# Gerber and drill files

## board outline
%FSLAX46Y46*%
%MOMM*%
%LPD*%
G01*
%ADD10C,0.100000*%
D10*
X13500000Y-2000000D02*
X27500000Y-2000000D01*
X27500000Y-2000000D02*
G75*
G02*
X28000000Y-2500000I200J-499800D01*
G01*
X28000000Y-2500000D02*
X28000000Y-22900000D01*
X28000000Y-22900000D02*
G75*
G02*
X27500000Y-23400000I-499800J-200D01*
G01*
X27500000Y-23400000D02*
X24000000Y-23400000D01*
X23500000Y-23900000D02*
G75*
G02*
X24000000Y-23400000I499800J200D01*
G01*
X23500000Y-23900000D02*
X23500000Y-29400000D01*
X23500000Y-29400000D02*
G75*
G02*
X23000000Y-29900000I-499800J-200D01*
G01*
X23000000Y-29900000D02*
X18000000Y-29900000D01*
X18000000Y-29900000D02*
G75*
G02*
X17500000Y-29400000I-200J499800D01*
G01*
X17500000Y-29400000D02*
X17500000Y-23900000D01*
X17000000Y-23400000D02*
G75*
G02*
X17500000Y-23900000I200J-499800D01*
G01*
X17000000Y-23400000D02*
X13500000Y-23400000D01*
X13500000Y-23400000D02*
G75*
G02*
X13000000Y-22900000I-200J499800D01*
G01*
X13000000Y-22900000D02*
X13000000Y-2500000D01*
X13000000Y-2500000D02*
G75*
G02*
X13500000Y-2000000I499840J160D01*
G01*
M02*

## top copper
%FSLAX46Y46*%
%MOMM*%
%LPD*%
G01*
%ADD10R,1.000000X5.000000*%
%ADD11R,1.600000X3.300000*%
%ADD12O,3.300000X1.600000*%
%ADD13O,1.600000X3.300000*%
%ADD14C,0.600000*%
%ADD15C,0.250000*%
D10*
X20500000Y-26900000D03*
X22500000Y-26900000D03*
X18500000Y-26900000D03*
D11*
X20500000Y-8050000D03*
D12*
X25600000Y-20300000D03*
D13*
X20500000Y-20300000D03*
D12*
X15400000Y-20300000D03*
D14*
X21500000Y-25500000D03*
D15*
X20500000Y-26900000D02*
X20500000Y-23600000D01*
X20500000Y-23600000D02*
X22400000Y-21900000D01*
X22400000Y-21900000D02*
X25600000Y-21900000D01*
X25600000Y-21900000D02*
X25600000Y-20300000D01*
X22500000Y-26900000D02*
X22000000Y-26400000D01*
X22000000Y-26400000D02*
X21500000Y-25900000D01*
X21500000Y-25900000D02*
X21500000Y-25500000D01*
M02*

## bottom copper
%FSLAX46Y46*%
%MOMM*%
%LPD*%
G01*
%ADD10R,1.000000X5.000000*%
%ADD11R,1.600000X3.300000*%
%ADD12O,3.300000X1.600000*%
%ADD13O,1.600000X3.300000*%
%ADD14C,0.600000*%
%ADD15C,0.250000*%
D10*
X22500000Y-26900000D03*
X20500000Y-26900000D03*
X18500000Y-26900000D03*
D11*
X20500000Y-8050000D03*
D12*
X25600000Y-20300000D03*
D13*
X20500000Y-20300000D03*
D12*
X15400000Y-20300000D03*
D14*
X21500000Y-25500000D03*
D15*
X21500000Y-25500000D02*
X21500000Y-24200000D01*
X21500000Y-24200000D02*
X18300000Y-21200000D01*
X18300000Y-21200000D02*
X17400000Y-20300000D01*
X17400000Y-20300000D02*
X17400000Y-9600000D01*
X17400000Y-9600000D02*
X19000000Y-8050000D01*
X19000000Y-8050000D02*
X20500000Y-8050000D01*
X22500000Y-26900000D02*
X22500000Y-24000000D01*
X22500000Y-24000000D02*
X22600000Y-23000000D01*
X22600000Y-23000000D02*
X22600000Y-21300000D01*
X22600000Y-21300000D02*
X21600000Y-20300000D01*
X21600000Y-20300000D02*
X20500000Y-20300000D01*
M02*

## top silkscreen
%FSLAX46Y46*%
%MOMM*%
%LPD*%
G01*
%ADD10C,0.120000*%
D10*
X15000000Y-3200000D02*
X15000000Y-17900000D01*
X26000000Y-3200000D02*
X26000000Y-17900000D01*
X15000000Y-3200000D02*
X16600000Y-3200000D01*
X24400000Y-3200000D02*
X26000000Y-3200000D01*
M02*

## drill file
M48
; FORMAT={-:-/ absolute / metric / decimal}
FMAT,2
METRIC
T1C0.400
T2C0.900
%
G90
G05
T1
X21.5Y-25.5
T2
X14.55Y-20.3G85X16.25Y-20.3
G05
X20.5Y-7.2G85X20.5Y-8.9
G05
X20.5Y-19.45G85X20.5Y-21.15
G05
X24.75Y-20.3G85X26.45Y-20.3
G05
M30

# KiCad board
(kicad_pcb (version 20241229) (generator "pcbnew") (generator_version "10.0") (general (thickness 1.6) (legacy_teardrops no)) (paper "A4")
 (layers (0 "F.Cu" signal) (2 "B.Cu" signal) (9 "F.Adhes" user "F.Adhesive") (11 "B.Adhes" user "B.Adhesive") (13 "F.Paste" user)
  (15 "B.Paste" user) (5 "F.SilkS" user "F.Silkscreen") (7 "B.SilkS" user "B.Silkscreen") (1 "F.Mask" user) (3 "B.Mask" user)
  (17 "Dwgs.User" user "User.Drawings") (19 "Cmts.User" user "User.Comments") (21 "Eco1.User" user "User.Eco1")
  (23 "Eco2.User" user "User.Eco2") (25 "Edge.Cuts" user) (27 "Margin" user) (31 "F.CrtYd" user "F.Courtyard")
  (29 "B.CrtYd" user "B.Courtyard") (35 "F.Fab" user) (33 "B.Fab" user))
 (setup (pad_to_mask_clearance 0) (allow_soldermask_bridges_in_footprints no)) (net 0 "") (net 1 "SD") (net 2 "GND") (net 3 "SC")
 (gr_line (start 13.5 2.0) (end 27.5 2.0) (stroke (width 0.1) (type default)) (layer "Edge.Cuts"))
 (gr_arc (start 27.5 2.0) (mid 27.8536 2.1464) (end 28.0 2.5) (stroke (width 0.1) (type default)) (layer "Edge.Cuts"))
 (gr_line (start 28.0 2.5) (end 28.0 22.9) (stroke (width 0.1) (type default)) (layer "Edge.Cuts"))
 (gr_arc (start 28.0 22.9) (mid 27.8536 23.2536) (end 27.5 23.4) (stroke (width 0.1) (type default)) (layer "Edge.Cuts"))
 (gr_line (start 27.5 23.4) (end 24.0 23.4) (stroke (width 0.1) (type default)) (layer "Edge.Cuts"))
 (gr_arc (start 24.0 23.4) (mid 23.6464 23.5464) (end 23.5 23.9) (stroke (width 0.1) (type default)) (layer "Edge.Cuts"))
 (gr_line (start 23.5 23.9) (end 23.5 29.4) (stroke (width 0.1) (type default)) (layer "Edge.Cuts"))
 (gr_arc (start 23.5 29.4) (mid 23.3536 29.7536) (end 23.0 29.9) (stroke (width 0.1) (type default)) (layer "Edge.Cuts"))
 (gr_line (start 23.0 29.9) (end 18.0 29.9) (stroke (width 0.1) (type default)) (layer "Edge.Cuts"))
 (gr_arc (start 18.0 29.9) (mid 17.6464 29.7536) (end 17.5 29.4) (stroke (width 0.1) (type default)) (layer "Edge.Cuts"))
 (gr_line (start 17.5 29.4) (end 17.5 23.9) (stroke (width 0.1) (type default)) (layer "Edge.Cuts"))
 (gr_arc (start 17.5 23.9) (mid 17.3536 23.5464) (end 17.0 23.4) (stroke (width 0.1) (type default)) (layer "Edge.Cuts"))
 (gr_line (start 17.0 23.4) (end 13.5 23.4) (stroke (width 0.1) (type default)) (layer "Edge.Cuts"))
 (gr_arc (start 13.5 23.4) (mid 13.1464 23.2536) (end 13.0 22.9) (stroke (width 0.1) (type default)) (layer "Edge.Cuts"))
 (gr_line (start 13.0 22.9) (end 13.0 2.5) (stroke (width 0.1) (type default)) (layer "Edge.Cuts"))
 (gr_arc (start 13.0 2.5) (mid 13.1464 2.1464) (end 13.5 2.0) (stroke (width 0.1) (type default)) (layer "Edge.Cuts"))
 (gr_line (start 15.0 3.2) (end 15.0 17.9) (stroke (width 0.12) (type default)) (layer "F.SilkS"))
 (gr_line (start 26.0 3.2) (end 26.0 17.9) (stroke (width 0.12) (type default)) (layer "F.SilkS"))
 (gr_line (start 15.0 3.2) (end 16.6 3.2) (stroke (width 0.12) (type default)) (layer "F.SilkS"))
 (gr_line (start 24.4 3.2) (end 26.0 3.2) (stroke (width 0.12) (type default)) (layer "F.SilkS"))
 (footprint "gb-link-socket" (layer "F.Cu") (at 20.5 26.9)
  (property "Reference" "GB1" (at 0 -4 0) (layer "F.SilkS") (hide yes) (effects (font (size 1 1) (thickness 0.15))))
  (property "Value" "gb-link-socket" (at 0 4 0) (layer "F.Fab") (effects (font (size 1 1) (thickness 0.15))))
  (pad "4" smd rect (at 0 0) (size 1 5) (layers "F.Cu" "F.Mask") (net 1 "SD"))
  (pad "6" smd rect (at 2 0) (size 1 5) (layers "F.Cu" "F.Mask") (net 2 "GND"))
  (pad "2" smd rect (at -2 0) (size 1 5) (layers "F.Cu" "F.Mask"))
  (pad "5" smd rect (at 2 0) (size 1 5) (layers "B.Cu" "B.Mask") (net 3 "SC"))
  (pad "3" smd rect (at 0 0) (size 1 5) (layers "B.Cu" "B.Mask"))
  (pad "1" smd rect (at -2 0) (size 1 5) (layers "B.Cu" "B.Mask")))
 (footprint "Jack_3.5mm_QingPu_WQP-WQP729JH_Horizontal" (layer "F.Cu") (at 20.5 2.0 270)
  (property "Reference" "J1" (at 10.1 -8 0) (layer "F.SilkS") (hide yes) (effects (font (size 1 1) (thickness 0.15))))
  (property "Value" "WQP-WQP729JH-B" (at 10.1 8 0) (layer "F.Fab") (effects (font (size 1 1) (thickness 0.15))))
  (pad "1" thru_hole rect (at 6.05 0) (size 1.6 3.3) (drill oval 0.9 2.6) (layers "*.Cu" "*.Mask") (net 2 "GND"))
  (pad "2" thru_hole oval (at 18.3 -5.1) (size 3.3 1.6) (drill oval 2.6 0.9) (layers "*.Cu" "*.Mask") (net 1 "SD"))
  (pad "3" thru_hole oval (at 18.3 0) (size 1.6 3.3) (drill oval 0.9 2.6) (layers "*.Cu" "*.Mask") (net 3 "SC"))
  (pad "4" thru_hole oval (at 18.3 5.1) (size 3.3 1.6) (drill oval 2.6 0.9) (layers "*.Cu" "*.Mask")))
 (segment (start 20.5 26.9) (end 20.5 23.6) (width 0.25) (layer "F.Cu") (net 1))
 (segment (start 20.5 23.6) (end 22.4 21.9) (width 0.25) (layer "F.Cu") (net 1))
 (segment (start 22.4 21.9) (end 25.6 21.9) (width 0.25) (layer "F.Cu") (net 1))
 (segment (start 25.6 21.9) (end 25.6 20.3) (width 0.25) (layer "F.Cu") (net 1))
 (segment (start 22.5 26.9) (end 22.0 26.4) (width 0.25) (layer "F.Cu") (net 2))
 (segment (start 22.0 26.4) (end 21.5 25.9) (width 0.25) (layer "F.Cu") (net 2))
 (segment (start 21.5 25.9) (end 21.5 25.5) (width 0.25) (layer "F.Cu") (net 2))
 (via (at 21.5 25.5) (size 0.6) (drill 0.4) (layers "F.Cu" "B.Cu") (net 2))
 (segment (start 21.5 25.5) (end 21.5 24.2) (width 0.25) (layer "B.Cu") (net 2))
 (segment (start 21.5 24.2) (end 18.3 21.2) (width 0.25) (layer "B.Cu") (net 2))
 (segment (start 18.3 21.2) (end 17.4 20.3) (width 0.25) (layer "B.Cu") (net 2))
 (segment (start 17.4 20.3) (end 17.4 9.6) (width 0.25) (layer "B.Cu") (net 2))
 (segment (start 17.4 9.6) (end 19.0 8.05) (width 0.25) (layer "B.Cu") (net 2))
 (segment (start 19.0 8.05) (end 20.5 8.05) (width 0.25) (layer "B.Cu") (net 2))
 (segment (start 22.5 26.9) (end 22.5 24.0) (width 0.25) (layer "B.Cu") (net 3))
 (segment (start 22.5 24.0) (end 22.6 23.0) (width 0.25) (layer "B.Cu") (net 3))
 (segment (start 22.6 23.0) (end 22.6 21.3) (width 0.25) (layer "B.Cu") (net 3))
 (segment (start 22.6 21.3) (end 21.6 20.3) (width 0.25) (layer "B.Cu") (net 3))
 (segment (start 21.6 20.3) (end 20.5 20.3) (width 0.25) (layer "B.Cu") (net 3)))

